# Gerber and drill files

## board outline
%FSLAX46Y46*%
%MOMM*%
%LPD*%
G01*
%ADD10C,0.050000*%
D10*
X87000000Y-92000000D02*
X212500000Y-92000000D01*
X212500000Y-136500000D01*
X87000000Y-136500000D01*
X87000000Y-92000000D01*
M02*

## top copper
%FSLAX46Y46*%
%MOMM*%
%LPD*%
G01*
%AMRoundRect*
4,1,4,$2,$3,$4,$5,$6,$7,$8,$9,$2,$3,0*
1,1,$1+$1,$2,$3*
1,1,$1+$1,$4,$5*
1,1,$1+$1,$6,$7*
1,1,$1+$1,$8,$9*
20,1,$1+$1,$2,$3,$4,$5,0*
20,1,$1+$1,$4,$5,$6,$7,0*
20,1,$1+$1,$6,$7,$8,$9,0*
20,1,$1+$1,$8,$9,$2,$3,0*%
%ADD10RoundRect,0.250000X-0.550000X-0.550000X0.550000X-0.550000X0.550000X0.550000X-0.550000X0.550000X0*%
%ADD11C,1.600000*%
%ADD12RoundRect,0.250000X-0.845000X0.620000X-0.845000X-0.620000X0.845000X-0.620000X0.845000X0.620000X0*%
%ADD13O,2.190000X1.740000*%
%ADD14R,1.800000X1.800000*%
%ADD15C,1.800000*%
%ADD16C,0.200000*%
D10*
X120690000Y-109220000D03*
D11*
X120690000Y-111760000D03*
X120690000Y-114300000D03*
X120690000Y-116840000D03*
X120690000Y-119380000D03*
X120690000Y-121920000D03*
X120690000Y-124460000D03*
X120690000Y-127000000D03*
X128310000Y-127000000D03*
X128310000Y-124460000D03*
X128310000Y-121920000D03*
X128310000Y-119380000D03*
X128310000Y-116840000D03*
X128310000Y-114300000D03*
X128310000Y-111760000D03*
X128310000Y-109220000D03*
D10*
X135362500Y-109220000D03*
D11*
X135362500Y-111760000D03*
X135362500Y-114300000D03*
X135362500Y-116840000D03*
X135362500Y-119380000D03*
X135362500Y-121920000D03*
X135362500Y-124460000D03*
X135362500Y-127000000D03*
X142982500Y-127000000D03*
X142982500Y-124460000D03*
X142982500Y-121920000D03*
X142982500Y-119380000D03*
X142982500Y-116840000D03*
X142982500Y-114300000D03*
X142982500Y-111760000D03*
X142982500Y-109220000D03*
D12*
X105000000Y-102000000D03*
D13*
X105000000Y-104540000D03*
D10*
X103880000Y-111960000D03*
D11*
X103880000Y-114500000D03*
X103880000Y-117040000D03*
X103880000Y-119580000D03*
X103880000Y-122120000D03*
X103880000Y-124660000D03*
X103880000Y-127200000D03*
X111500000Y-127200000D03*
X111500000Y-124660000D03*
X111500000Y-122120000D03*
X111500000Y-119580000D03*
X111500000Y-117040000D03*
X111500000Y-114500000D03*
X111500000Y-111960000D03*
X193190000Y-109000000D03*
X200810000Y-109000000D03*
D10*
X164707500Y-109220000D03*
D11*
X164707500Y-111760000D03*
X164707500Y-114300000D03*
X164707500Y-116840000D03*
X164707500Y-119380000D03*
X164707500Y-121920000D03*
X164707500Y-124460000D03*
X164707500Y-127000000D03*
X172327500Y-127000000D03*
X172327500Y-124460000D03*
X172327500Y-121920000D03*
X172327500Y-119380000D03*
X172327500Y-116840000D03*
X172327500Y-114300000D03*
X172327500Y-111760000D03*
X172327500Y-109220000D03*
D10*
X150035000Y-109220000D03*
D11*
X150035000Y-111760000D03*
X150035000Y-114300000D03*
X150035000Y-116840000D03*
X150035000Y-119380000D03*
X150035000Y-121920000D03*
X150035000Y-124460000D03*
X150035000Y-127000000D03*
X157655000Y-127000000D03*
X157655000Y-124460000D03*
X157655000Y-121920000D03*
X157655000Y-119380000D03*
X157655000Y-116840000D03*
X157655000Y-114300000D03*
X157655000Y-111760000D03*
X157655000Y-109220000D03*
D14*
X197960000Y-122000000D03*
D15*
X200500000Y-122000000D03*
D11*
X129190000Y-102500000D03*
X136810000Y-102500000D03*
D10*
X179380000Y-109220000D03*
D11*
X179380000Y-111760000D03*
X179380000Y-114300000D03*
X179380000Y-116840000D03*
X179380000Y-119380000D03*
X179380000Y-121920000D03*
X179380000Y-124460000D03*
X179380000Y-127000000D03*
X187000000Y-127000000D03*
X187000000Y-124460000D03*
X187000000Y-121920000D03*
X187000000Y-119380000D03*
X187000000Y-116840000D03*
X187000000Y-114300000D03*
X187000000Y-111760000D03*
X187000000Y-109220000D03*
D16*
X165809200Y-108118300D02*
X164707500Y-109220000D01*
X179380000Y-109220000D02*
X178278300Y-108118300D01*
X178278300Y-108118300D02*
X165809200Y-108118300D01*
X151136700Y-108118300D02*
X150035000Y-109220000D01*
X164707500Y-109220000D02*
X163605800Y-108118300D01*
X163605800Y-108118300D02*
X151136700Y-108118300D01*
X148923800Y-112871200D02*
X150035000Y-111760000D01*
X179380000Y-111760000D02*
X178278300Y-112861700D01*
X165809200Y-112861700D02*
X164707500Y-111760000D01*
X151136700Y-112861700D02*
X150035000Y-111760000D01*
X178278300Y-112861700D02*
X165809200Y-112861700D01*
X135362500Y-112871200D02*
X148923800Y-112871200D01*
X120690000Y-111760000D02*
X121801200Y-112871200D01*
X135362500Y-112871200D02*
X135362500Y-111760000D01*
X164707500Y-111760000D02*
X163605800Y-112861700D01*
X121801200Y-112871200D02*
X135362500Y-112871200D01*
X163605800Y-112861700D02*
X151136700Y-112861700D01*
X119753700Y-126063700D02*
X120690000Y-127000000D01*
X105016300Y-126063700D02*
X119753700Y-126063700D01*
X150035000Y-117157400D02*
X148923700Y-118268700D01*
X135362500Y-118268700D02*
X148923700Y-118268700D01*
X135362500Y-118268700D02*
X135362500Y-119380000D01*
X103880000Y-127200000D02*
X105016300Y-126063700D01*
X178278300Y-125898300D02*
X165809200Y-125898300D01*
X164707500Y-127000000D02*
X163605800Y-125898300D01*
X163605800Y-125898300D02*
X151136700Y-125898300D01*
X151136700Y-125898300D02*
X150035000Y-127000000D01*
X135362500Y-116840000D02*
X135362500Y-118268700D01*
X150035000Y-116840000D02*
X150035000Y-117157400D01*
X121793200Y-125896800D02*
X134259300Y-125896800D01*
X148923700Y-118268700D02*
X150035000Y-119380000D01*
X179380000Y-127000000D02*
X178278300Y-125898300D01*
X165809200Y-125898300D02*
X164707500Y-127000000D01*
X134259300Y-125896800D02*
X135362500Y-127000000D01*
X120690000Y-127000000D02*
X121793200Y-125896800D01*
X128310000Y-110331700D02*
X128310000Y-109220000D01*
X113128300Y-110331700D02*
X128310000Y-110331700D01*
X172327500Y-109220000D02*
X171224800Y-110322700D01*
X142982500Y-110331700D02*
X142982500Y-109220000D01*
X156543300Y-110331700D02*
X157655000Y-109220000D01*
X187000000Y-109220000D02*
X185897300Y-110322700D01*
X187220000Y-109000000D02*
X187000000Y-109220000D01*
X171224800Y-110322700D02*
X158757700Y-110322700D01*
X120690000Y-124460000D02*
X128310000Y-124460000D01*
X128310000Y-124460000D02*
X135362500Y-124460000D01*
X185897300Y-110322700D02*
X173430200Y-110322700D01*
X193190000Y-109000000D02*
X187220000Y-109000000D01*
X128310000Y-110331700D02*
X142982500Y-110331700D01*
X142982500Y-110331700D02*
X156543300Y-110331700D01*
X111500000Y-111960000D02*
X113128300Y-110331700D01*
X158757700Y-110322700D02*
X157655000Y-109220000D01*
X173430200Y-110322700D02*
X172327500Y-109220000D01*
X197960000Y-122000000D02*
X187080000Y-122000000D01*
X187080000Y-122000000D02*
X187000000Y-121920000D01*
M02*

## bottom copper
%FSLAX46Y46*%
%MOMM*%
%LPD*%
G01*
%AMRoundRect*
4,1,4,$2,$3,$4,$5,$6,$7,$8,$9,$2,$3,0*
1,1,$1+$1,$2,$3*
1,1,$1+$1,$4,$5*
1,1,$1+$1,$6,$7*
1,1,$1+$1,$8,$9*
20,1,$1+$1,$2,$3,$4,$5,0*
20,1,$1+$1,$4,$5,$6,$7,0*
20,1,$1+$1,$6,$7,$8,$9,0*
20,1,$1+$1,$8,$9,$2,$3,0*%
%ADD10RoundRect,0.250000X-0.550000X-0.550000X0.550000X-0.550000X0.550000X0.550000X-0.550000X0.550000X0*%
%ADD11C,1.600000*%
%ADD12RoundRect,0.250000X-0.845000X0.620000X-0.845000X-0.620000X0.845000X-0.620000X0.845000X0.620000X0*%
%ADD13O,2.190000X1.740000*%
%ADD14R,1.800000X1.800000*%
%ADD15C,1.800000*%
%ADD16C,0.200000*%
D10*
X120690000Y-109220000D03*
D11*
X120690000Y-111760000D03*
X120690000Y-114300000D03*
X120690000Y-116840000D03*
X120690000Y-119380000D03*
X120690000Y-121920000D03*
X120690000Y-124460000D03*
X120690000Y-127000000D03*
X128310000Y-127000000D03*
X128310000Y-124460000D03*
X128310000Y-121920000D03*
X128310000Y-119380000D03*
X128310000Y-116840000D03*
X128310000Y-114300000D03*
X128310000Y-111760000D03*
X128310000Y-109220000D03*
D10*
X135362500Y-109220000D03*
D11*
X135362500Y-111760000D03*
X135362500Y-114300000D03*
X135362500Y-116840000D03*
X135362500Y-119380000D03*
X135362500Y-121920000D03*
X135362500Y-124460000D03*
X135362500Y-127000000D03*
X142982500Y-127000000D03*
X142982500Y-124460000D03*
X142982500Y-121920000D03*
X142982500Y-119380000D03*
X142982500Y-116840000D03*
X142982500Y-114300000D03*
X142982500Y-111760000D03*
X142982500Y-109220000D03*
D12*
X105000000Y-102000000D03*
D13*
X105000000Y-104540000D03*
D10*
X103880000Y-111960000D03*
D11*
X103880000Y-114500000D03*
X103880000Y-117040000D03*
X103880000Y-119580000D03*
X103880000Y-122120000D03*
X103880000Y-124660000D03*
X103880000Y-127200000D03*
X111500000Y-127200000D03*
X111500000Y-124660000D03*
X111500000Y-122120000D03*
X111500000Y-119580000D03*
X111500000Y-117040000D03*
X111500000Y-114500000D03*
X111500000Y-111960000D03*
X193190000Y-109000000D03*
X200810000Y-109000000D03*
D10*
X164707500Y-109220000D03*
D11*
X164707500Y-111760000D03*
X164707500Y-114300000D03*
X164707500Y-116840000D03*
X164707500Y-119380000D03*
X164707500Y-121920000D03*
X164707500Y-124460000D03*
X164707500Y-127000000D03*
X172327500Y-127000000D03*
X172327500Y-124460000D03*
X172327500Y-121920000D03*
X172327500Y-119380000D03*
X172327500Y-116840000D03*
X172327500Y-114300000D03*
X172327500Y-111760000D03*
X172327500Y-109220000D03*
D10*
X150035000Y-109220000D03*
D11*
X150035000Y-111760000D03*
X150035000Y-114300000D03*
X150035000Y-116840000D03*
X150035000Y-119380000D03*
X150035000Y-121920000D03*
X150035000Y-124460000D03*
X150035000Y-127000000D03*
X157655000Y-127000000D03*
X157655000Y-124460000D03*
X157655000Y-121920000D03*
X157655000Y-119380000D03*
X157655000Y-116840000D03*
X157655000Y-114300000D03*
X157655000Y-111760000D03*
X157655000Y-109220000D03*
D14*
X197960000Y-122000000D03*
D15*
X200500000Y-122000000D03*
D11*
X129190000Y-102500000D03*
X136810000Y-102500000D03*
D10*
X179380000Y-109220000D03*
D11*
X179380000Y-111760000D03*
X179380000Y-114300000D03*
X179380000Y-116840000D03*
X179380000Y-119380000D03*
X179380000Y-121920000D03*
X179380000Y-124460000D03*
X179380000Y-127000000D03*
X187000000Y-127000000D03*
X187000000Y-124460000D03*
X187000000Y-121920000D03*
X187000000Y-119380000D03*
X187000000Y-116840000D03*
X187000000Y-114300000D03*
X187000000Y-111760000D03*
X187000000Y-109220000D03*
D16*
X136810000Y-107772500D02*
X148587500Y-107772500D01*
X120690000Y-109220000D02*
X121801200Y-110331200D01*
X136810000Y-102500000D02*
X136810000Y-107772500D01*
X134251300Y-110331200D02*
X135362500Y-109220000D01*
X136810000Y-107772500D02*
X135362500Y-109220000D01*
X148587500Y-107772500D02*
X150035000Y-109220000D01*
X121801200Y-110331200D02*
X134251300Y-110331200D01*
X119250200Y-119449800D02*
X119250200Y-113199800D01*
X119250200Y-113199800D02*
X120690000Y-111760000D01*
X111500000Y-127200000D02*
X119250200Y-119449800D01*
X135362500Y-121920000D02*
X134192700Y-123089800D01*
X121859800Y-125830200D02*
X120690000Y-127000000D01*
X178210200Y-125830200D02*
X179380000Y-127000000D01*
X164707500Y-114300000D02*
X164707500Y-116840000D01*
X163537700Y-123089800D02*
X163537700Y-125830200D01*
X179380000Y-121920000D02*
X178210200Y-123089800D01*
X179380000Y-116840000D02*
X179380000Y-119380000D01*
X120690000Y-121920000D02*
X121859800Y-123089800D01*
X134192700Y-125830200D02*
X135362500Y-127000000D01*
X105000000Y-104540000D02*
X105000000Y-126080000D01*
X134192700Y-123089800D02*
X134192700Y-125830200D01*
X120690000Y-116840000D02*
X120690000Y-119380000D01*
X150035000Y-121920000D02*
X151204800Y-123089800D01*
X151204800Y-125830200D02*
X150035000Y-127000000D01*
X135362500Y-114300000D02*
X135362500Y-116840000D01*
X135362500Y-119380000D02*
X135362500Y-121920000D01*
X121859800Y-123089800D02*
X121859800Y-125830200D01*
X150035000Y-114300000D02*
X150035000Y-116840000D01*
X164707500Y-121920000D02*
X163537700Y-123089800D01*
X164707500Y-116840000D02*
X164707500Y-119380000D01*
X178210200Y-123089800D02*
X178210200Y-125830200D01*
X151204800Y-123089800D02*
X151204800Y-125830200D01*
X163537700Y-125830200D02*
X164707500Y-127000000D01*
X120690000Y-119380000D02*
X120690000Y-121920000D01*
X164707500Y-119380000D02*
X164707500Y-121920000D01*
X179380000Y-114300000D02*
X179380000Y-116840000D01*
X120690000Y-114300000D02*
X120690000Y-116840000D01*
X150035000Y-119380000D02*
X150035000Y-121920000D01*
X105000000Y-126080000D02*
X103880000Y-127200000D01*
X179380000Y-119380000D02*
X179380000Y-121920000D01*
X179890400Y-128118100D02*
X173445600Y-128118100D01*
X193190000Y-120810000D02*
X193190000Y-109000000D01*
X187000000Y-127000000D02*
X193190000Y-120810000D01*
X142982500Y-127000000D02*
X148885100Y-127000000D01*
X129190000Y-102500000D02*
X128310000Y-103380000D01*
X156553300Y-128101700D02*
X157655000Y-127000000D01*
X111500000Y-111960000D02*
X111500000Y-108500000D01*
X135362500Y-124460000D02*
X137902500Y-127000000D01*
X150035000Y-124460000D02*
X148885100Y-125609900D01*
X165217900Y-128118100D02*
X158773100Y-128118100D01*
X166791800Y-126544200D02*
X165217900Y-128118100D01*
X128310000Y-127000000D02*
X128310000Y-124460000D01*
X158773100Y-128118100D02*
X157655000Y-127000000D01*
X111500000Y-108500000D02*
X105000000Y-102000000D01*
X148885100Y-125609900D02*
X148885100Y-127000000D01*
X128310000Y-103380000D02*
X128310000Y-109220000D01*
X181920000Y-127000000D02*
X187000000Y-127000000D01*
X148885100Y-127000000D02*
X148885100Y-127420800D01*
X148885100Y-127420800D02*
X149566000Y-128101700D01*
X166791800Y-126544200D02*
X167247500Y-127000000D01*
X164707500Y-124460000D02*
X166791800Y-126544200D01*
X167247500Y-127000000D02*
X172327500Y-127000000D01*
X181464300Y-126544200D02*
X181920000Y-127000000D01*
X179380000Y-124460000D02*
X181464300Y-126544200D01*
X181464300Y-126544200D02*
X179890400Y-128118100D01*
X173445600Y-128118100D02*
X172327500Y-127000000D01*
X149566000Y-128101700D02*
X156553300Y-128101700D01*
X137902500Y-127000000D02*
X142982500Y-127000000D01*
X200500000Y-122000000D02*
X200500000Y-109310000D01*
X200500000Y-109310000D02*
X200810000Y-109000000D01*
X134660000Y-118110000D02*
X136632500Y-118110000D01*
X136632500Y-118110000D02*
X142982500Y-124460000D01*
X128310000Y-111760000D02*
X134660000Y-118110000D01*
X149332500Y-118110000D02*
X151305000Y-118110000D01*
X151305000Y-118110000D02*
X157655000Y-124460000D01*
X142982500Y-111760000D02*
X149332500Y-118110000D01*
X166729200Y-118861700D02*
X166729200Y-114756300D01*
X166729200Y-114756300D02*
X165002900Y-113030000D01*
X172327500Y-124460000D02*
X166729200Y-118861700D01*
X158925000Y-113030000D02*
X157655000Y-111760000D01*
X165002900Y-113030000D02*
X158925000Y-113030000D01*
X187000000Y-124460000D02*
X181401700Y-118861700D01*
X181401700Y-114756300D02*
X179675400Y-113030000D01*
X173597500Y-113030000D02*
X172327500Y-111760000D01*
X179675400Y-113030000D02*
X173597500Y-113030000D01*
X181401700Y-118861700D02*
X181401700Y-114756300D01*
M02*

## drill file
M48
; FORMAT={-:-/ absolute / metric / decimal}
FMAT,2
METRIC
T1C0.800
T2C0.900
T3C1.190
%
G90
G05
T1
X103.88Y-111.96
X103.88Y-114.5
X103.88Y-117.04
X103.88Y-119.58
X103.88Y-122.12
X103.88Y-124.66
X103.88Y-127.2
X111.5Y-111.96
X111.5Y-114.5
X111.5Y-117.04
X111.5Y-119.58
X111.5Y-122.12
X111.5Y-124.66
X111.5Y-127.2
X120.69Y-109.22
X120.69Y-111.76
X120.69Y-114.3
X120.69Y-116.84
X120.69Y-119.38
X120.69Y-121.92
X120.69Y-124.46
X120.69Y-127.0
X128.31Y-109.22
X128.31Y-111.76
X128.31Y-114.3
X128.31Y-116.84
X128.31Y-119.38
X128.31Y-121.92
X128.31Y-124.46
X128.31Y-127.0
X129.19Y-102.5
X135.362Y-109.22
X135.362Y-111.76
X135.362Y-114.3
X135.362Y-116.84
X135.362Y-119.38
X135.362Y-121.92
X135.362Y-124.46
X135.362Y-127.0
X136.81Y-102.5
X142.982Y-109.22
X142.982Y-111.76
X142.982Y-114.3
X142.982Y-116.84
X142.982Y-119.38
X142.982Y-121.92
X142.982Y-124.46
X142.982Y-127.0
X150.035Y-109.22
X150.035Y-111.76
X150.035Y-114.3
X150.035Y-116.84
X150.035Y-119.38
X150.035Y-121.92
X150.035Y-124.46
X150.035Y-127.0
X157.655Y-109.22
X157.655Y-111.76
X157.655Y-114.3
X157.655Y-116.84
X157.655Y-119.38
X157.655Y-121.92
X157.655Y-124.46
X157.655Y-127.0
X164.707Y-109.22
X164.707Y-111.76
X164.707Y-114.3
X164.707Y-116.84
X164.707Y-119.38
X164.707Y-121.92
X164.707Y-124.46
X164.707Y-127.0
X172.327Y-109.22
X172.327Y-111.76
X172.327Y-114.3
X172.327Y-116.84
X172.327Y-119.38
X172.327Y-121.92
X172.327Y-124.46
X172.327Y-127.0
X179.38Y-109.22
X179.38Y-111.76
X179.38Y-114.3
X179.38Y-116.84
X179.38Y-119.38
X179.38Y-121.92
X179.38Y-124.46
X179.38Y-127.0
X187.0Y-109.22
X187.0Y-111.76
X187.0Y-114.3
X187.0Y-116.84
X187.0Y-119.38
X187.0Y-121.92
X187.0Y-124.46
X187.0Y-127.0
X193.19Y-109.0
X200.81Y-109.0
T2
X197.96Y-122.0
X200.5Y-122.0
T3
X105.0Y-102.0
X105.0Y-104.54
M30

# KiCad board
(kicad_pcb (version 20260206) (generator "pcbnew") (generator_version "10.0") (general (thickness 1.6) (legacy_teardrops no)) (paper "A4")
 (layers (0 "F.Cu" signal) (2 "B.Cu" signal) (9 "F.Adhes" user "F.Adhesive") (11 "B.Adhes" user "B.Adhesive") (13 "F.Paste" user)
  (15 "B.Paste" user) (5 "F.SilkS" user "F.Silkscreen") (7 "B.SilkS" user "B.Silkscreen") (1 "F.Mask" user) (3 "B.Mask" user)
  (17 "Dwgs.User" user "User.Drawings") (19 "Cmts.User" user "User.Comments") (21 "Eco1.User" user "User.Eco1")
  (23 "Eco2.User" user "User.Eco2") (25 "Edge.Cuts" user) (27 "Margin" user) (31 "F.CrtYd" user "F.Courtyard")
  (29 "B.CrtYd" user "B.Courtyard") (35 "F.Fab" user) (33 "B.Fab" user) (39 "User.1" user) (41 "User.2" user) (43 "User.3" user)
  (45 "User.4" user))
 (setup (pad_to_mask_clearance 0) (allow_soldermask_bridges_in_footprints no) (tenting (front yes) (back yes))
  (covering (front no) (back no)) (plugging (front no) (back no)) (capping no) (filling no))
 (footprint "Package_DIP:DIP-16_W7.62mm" (layer "F.Cu") (at 120.69 109.22)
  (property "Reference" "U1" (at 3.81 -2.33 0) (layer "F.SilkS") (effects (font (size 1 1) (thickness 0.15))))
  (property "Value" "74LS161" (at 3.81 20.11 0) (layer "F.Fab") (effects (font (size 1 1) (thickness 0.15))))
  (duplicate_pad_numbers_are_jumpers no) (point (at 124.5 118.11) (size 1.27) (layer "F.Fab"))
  (pad "1" thru_hole roundrect (at 0 0) (size 1.6 1.6) (drill 0.8) (layers "*.Cu" "*.Mask") (remove_unused_layers no)
   (roundrect_rratio 0.15625) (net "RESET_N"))
  (pad "2" thru_hole circle (at 0 2.54) (size 1.6 1.6) (drill 0.8) (layers "*.Cu" "*.Mask") (remove_unused_layers no) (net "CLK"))
  (pad "3" thru_hole circle (at 0 5.08) (size 1.6 1.6) (drill 0.8) (layers "*.Cu" "*.Mask") (remove_unused_layers no) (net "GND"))
  (pad "4" thru_hole circle (at 0 7.62) (size 1.6 1.6) (drill 0.8) (layers "*.Cu" "*.Mask") (remove_unused_layers no) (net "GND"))
  (pad "5" thru_hole circle (at 0 10.16) (size 1.6 1.6) (drill 0.8) (layers "*.Cu" "*.Mask") (remove_unused_layers no) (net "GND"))
  (pad "6" thru_hole circle (at 0 12.7) (size 1.6 1.6) (drill 0.8) (layers "*.Cu" "*.Mask") (remove_unused_layers no) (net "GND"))
  (pad "7" thru_hole circle (at 0 15.24) (size 1.6 1.6) (drill 0.8) (layers "*.Cu" "*.Mask") (remove_unused_layers no) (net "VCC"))
  (pad "8" thru_hole circle (at 0 17.78) (size 1.6 1.6) (drill 0.8) (layers "*.Cu" "*.Mask") (remove_unused_layers no) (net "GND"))
  (pad "9" thru_hole circle (at 7.62 17.78) (size 1.6 1.6) (drill 0.8) (layers "*.Cu" "*.Mask") (remove_unused_layers no) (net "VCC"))
  (pad "10" thru_hole circle (at 7.62 15.24) (size 1.6 1.6) (drill 0.8) (layers "*.Cu" "*.Mask") (remove_unused_layers no) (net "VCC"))
  (pad "11" thru_hole circle (at 7.62 12.7) (size 1.6 1.6) (drill 0.8) (layers "*.Cu" "*.Mask") (remove_unused_layers no) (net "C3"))
  (pad "12" thru_hole circle (at 7.62 10.16) (size 1.6 1.6) (drill 0.8) (layers "*.Cu" "*.Mask") (remove_unused_layers no) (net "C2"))
  (pad "13" thru_hole circle (at 7.62 7.62) (size 1.6 1.6) (drill 0.8) (layers "*.Cu" "*.Mask") (remove_unused_layers no) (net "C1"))
  (pad "14" thru_hole circle (at 7.62 5.08) (size 1.6 1.6) (drill 0.8) (layers "*.Cu" "*.Mask") (remove_unused_layers no) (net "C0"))
  (pad "15" thru_hole circle (at 7.62 2.54) (size 1.6 1.6) (drill 0.8) (layers "*.Cu" "*.Mask") (remove_unused_layers no) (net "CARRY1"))
  (pad "16" thru_hole circle (at 7.62 0) (size 1.6 1.6) (drill 0.8) (layers "*.Cu" "*.Mask") (remove_unused_layers no) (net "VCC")))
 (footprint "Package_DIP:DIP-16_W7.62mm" (layer "F.Cu") (at 135.3625 109.22)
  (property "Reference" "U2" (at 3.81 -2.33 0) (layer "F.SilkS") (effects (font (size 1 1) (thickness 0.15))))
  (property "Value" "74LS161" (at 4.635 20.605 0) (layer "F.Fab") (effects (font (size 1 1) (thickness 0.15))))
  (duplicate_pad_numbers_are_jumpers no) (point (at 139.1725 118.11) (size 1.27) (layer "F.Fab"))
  (pad "1" thru_hole roundrect (at 0 0) (size 1.6 1.6) (drill 0.8) (layers "*.Cu" "*.Mask") (remove_unused_layers no)
   (roundrect_rratio 0.15625) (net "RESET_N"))
  (pad "2" thru_hole circle (at 0 2.54) (size 1.6 1.6) (drill 0.8) (layers "*.Cu" "*.Mask") (remove_unused_layers no) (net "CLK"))
  (pad "3" thru_hole circle (at 0 5.08) (size 1.6 1.6) (drill 0.8) (layers "*.Cu" "*.Mask") (remove_unused_layers no) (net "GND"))
  (pad "4" thru_hole circle (at 0 7.62) (size 1.6 1.6) (drill 0.8) (layers "*.Cu" "*.Mask") (remove_unused_layers no) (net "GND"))
  (pad "5" thru_hole circle (at 0 10.16) (size 1.6 1.6) (drill 0.8) (layers "*.Cu" "*.Mask") (remove_unused_layers no) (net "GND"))
  (pad "6" thru_hole circle (at 0 12.7) (size 1.6 1.6) (drill 0.8) (layers "*.Cu" "*.Mask") (remove_unused_layers no) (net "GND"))
  (pad "7" thru_hole circle (at 0 15.24) (size 1.6 1.6) (drill 0.8) (layers "*.Cu" "*.Mask") (remove_unused_layers no) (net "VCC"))
  (pad "8" thru_hole circle (at 0 17.78) (size 1.6 1.6) (drill 0.8) (layers "*.Cu" "*.Mask") (remove_unused_layers no) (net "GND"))
  (pad "9" thru_hole circle (at 7.62 17.78) (size 1.6 1.6) (drill 0.8) (layers "*.Cu" "*.Mask") (remove_unused_layers no) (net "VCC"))
  (pad "10" thru_hole circle (at 7.62 15.24) (size 1.6 1.6) (drill 0.8) (layers "*.Cu" "*.Mask") (remove_unused_layers no) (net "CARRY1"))
  (pad "11" thru_hole circle (at 7.62 12.7) (size 1.6 1.6) (drill 0.8) (layers "*.Cu" "*.Mask") (remove_unused_layers no) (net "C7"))
  (pad "12" thru_hole circle (at 7.62 10.16) (size 1.6 1.6) (drill 0.8) (layers "*.Cu" "*.Mask") (remove_unused_layers no) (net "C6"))
  (pad "13" thru_hole circle (at 7.62 7.62) (size 1.6 1.6) (drill 0.8) (layers "*.Cu" "*.Mask") (remove_unused_layers no) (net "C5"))
  (pad "14" thru_hole circle (at 7.62 5.08) (size 1.6 1.6) (drill 0.8) (layers "*.Cu" "*.Mask") (remove_unused_layers no) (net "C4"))
  (pad "15" thru_hole circle (at 7.62 2.54) (size 1.6 1.6) (drill 0.8) (layers "*.Cu" "*.Mask") (remove_unused_layers no) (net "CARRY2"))
  (pad "16" thru_hole circle (at 7.62 0) (size 1.6 1.6) (drill 0.8) (layers "*.Cu" "*.Mask") (remove_unused_layers no) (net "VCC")))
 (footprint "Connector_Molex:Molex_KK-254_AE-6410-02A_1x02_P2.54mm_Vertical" (layer "F.Cu") (at 105 102 -90)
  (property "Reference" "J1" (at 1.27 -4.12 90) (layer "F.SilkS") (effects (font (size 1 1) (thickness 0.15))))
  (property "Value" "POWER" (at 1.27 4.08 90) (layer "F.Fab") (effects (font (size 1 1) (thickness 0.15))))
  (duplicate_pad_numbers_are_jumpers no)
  (pad "1" thru_hole roundrect (at 0 0 270) (size 1.74 2.19) (drill 1.19) (layers "*.Cu" "*.Mask") (remove_unused_layers no)
   (roundrect_rratio 0.143678) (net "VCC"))
  (pad "2" thru_hole oval (at 2.54 0 270) (size 1.74 2.19) (drill 1.19) (layers "*.Cu" "*.Mask") (remove_unused_layers no) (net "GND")))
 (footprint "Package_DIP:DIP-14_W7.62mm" (layer "F.Cu") (at 103.88 111.96)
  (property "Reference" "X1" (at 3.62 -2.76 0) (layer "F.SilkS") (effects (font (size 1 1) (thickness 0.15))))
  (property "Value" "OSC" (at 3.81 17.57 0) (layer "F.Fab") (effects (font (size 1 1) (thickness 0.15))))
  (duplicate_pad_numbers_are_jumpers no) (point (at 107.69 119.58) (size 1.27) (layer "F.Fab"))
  (pad "1" thru_hole roundrect (at 0 0) (size 1.6 1.6) (drill 0.8) (layers "*.Cu" "*.Mask") (remove_unused_layers no)
   (roundrect_rratio 0.15625))
  (pad "2" thru_hole circle (at 0 2.54) (size 1.6 1.6) (drill 0.8) (layers "*.Cu" "*.Mask") (remove_unused_layers no))
  (pad "3" thru_hole circle (at 0 5.08) (size 1.6 1.6) (drill 0.8) (layers "*.Cu" "*.Mask") (remove_unused_layers no))
  (pad "4" thru_hole circle (at 0 7.62) (size 1.6 1.6) (drill 0.8) (layers "*.Cu" "*.Mask") (remove_unused_layers no))
  (pad "5" thru_hole circle (at 0 10.16) (size 1.6 1.6) (drill 0.8) (layers "*.Cu" "*.Mask") (remove_unused_layers no))
  (pad "6" thru_hole circle (at 0 12.7) (size 1.6 1.6) (drill 0.8) (layers "*.Cu" "*.Mask") (remove_unused_layers no))
  (pad "7" thru_hole circle (at 0 15.24) (size 1.6 1.6) (drill 0.8) (layers "*.Cu" "*.Mask") (remove_unused_layers no) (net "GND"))
  (pad "8" thru_hole circle (at 7.62 15.24) (size 1.6 1.6) (drill 0.8) (layers "*.Cu" "*.Mask") (remove_unused_layers no) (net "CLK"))
  (pad "9" thru_hole circle (at 7.62 12.7) (size 1.6 1.6) (drill 0.8) (layers "*.Cu" "*.Mask") (remove_unused_layers no))
  (pad "10" thru_hole circle (at 7.62 10.16) (size 1.6 1.6) (drill 0.8) (layers "*.Cu" "*.Mask") (remove_unused_layers no))
  (pad "11" thru_hole circle (at 7.62 7.62) (size 1.6 1.6) (drill 0.8) (layers "*.Cu" "*.Mask") (remove_unused_layers no))
  (pad "12" thru_hole circle (at 7.62 5.08) (size 1.6 1.6) (drill 0.8) (layers "*.Cu" "*.Mask") (remove_unused_layers no))
  (pad "13" thru_hole circle (at 7.62 2.54) (size 1.6 1.6) (drill 0.8) (layers "*.Cu" "*.Mask") (remove_unused_layers no))
  (pad "14" thru_hole circle (at 7.62 0) (size 1.6 1.6) (drill 0.8) (layers "*.Cu" "*.Mask") (remove_unused_layers no) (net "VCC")))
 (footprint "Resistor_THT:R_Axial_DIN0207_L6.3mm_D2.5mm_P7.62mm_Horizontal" (layer "F.Cu") (at 193.19 109)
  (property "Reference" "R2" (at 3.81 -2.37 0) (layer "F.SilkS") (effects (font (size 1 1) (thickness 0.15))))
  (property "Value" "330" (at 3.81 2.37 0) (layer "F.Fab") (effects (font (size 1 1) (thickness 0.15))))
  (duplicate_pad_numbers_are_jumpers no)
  (pad "1" thru_hole circle (at 0 0) (size 1.6 1.6) (drill 0.8) (layers "*.Cu" "*.Mask") (remove_unused_layers no) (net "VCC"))
  (pad "2" thru_hole circle (at 7.62 0) (size 1.6 1.6) (drill 0.8) (layers "*.Cu" "*.Mask") (remove_unused_layers no) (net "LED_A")))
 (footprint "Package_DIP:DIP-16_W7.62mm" (layer "F.Cu") (at 164.7075 109.22)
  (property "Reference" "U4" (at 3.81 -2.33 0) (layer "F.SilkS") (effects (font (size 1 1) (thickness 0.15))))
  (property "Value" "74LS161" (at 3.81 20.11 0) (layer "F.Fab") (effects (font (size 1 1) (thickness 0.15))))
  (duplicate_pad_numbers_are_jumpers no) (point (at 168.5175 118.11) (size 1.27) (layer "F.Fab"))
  (pad "1" thru_hole roundrect (at 0 0) (size 1.6 1.6) (drill 0.8) (layers "*.Cu" "*.Mask") (remove_unused_layers no)
   (roundrect_rratio 0.15625) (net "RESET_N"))
  (pad "2" thru_hole circle (at 0 2.54) (size 1.6 1.6) (drill 0.8) (layers "*.Cu" "*.Mask") (remove_unused_layers no) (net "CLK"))
  (pad "3" thru_hole circle (at 0 5.08) (size 1.6 1.6) (drill 0.8) (layers "*.Cu" "*.Mask") (remove_unused_layers no) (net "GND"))
  (pad "4" thru_hole circle (at 0 7.62) (size 1.6 1.6) (drill 0.8) (layers "*.Cu" "*.Mask") (remove_unused_layers no) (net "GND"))
  (pad "5" thru_hole circle (at 0 10.16) (size 1.6 1.6) (drill 0.8) (layers "*.Cu" "*.Mask") (remove_unused_layers no) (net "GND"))
  (pad "6" thru_hole circle (at 0 12.7) (size 1.6 1.6) (drill 0.8) (layers "*.Cu" "*.Mask") (remove_unused_layers no) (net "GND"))
  (pad "7" thru_hole circle (at 0 15.24) (size 1.6 1.6) (drill 0.8) (layers "*.Cu" "*.Mask") (remove_unused_layers no) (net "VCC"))
  (pad "8" thru_hole circle (at 0 17.78) (size 1.6 1.6) (drill 0.8) (layers "*.Cu" "*.Mask") (remove_unused_layers no) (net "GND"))
  (pad "9" thru_hole circle (at 7.62 17.78) (size 1.6 1.6) (drill 0.8) (layers "*.Cu" "*.Mask") (remove_unused_layers no) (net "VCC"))
  (pad "10" thru_hole circle (at 7.62 15.24) (size 1.6 1.6) (drill 0.8) (layers "*.Cu" "*.Mask") (remove_unused_layers no) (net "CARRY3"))
  (pad "11" thru_hole circle (at 7.62 12.7) (size 1.6 1.6) (drill 0.8) (layers "*.Cu" "*.Mask") (remove_unused_layers no) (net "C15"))
  (pad "12" thru_hole circle (at 7.62 10.16) (size 1.6 1.6) (drill 0.8) (layers "*.Cu" "*.Mask") (remove_unused_layers no) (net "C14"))
  (pad "13" thru_hole circle (at 7.62 7.62) (size 1.6 1.6) (drill 0.8) (layers "*.Cu" "*.Mask") (remove_unused_layers no) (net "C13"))
  (pad "14" thru_hole circle (at 7.62 5.08) (size 1.6 1.6) (drill 0.8) (layers "*.Cu" "*.Mask") (remove_unused_layers no) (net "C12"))
  (pad "15" thru_hole circle (at 7.62 2.54) (size 1.6 1.6) (drill 0.8) (layers "*.Cu" "*.Mask") (remove_unused_layers no) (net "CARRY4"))
  (pad "16" thru_hole circle (at 7.62 0) (size 1.6 1.6) (drill 0.8) (layers "*.Cu" "*.Mask") (remove_unused_layers no) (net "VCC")))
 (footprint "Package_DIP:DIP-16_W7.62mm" (layer "F.Cu") (at 150.035 109.22)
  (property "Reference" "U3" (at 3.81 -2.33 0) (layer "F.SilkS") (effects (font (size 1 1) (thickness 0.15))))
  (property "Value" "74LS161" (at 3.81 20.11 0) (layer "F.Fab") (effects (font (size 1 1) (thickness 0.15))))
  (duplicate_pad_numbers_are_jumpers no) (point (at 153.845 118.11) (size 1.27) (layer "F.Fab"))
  (pad "1" thru_hole roundrect (at 0 0) (size 1.6 1.6) (drill 0.8) (layers "*.Cu" "*.Mask") (remove_unused_layers no)
   (roundrect_rratio 0.15625) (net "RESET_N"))
  (pad "2" thru_hole circle (at 0 2.54) (size 1.6 1.6) (drill 0.8) (layers "*.Cu" "*.Mask") (remove_unused_layers no) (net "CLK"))
  (pad "3" thru_hole circle (at 0 5.08) (size 1.6 1.6) (drill 0.8) (layers "*.Cu" "*.Mask") (remove_unused_layers no) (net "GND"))
  (pad "4" thru_hole circle (at 0 7.62) (size 1.6 1.6) (drill 0.8) (layers "*.Cu" "*.Mask") (remove_unused_layers no) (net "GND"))
  (pad "5" thru_hole circle (at 0 10.16) (size 1.6 1.6) (drill 0.8) (layers "*.Cu" "*.Mask") (remove_unused_layers no) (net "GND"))
  (pad "6" thru_hole circle (at 0 12.7) (size 1.6 1.6) (drill 0.8) (layers "*.Cu" "*.Mask") (remove_unused_layers no) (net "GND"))
  (pad "7" thru_hole circle (at 0 15.24) (size 1.6 1.6) (drill 0.8) (layers "*.Cu" "*.Mask") (remove_unused_layers no) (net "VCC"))
  (pad "8" thru_hole circle (at 0 17.78) (size 1.6 1.6) (drill 0.8) (layers "*.Cu" "*.Mask") (remove_unused_layers no) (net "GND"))
  (pad "9" thru_hole circle (at 7.62 17.78) (size 1.6 1.6) (drill 0.8) (layers "*.Cu" "*.Mask") (remove_unused_layers no) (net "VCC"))
  (pad "10" thru_hole circle (at 7.62 15.24) (size 1.6 1.6) (drill 0.8) (layers "*.Cu" "*.Mask") (remove_unused_layers no) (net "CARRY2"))
  (pad "11" thru_hole circle (at 7.62 12.7) (size 1.6 1.6) (drill 0.8) (layers "*.Cu" "*.Mask") (remove_unused_layers no) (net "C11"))
  (pad "12" thru_hole circle (at 7.62 10.16) (size 1.6 1.6) (drill 0.8) (layers "*.Cu" "*.Mask") (remove_unused_layers no) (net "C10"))
  (pad "13" thru_hole circle (at 7.62 7.62) (size 1.6 1.6) (drill 0.8) (layers "*.Cu" "*.Mask") (remove_unused_layers no) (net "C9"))
  (pad "14" thru_hole circle (at 7.62 5.08) (size 1.6 1.6) (drill 0.8) (layers "*.Cu" "*.Mask") (remove_unused_layers no) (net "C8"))
  (pad "15" thru_hole circle (at 7.62 2.54) (size 1.6 1.6) (drill 0.8) (layers "*.Cu" "*.Mask") (remove_unused_layers no) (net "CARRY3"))
  (pad "16" thru_hole circle (at 7.62 0) (size 1.6 1.6) (drill 0.8) (layers "*.Cu" "*.Mask") (remove_unused_layers no) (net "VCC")))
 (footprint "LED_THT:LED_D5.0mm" (layer "F.Cu") (at 197.96 122)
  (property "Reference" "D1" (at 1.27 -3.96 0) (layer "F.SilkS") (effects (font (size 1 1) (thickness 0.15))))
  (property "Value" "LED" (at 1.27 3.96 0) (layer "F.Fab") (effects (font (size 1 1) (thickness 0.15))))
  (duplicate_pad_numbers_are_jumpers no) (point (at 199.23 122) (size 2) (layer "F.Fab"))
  (pad "1" thru_hole rect (at 0 0) (size 1.8 1.8) (drill 0.9) (layers "*.Cu" "*.Mask") (remove_unused_layers no) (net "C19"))
  (pad "2" thru_hole circle (at 2.54 0) (size 1.8 1.8) (drill 0.9) (layers "*.Cu" "*.Mask") (remove_unused_layers no) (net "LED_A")))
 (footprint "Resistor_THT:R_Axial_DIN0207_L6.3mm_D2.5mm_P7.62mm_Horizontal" (layer "F.Cu") (at 129.19 102.5)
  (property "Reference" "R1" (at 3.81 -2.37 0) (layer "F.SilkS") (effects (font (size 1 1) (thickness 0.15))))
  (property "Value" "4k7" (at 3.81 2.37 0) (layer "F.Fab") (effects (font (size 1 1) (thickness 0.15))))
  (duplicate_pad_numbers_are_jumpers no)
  (pad "1" thru_hole circle (at 0 0) (size 1.6 1.6) (drill 0.8) (layers "*.Cu" "*.Mask") (remove_unused_layers no) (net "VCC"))
  (pad "2" thru_hole circle (at 7.62 0) (size 1.6 1.6) (drill 0.8) (layers "*.Cu" "*.Mask") (remove_unused_layers no) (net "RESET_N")))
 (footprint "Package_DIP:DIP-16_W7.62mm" (layer "F.Cu") (at 179.38 109.22)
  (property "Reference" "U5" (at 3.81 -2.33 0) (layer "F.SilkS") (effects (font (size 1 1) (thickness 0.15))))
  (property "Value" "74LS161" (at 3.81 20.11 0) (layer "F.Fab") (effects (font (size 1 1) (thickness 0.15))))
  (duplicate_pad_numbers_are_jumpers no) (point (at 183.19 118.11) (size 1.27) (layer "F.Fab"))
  (pad "1" thru_hole roundrect (at 0 0) (size 1.6 1.6) (drill 0.8) (layers "*.Cu" "*.Mask") (remove_unused_layers no)
   (roundrect_rratio 0.15625) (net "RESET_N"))
  (pad "2" thru_hole circle (at 0 2.54) (size 1.6 1.6) (drill 0.8) (layers "*.Cu" "*.Mask") (remove_unused_layers no) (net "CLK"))
  (pad "3" thru_hole circle (at 0 5.08) (size 1.6 1.6) (drill 0.8) (layers "*.Cu" "*.Mask") (remove_unused_layers no) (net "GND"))
  (pad "4" thru_hole circle (at 0 7.62) (size 1.6 1.6) (drill 0.8) (layers "*.Cu" "*.Mask") (remove_unused_layers no) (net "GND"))
  (pad "5" thru_hole circle (at 0 10.16) (size 1.6 1.6) (drill 0.8) (layers "*.Cu" "*.Mask") (remove_unused_layers no) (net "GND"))
  (pad "6" thru_hole circle (at 0 12.7) (size 1.6 1.6) (drill 0.8) (layers "*.Cu" "*.Mask") (remove_unused_layers no) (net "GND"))
  (pad "7" thru_hole circle (at 0 15.24) (size 1.6 1.6) (drill 0.8) (layers "*.Cu" "*.Mask") (remove_unused_layers no) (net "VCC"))
  (pad "8" thru_hole circle (at 0 17.78) (size 1.6 1.6) (drill 0.8) (layers "*.Cu" "*.Mask") (remove_unused_layers no) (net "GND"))
  (pad "9" thru_hole circle (at 7.62 17.78) (size 1.6 1.6) (drill 0.8) (layers "*.Cu" "*.Mask") (remove_unused_layers no) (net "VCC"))
  (pad "10" thru_hole circle (at 7.62 15.24) (size 1.6 1.6) (drill 0.8) (layers "*.Cu" "*.Mask") (remove_unused_layers no) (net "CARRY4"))
  (pad "11" thru_hole circle (at 7.62 12.7) (size 1.6 1.6) (drill 0.8) (layers "*.Cu" "*.Mask") (remove_unused_layers no) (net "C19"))
  (pad "12" thru_hole circle (at 7.62 10.16) (size 1.6 1.6) (drill 0.8) (layers "*.Cu" "*.Mask") (remove_unused_layers no) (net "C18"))
  (pad "13" thru_hole circle (at 7.62 7.62) (size 1.6 1.6) (drill 0.8) (layers "*.Cu" "*.Mask") (remove_unused_layers no) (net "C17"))
  (pad "14" thru_hole circle (at 7.62 5.08) (size 1.6 1.6) (drill 0.8) (layers "*.Cu" "*.Mask") (remove_unused_layers no) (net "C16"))
  (pad "15" thru_hole circle (at 7.62 2.54) (size 1.6 1.6) (drill 0.8) (layers "*.Cu" "*.Mask") (remove_unused_layers no))
  (pad "16" thru_hole circle (at 7.62 0) (size 1.6 1.6) (drill 0.8) (layers "*.Cu" "*.Mask") (remove_unused_layers no) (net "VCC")))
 (gr_rect (start 87 92) (end 212.5 136.5) (stroke (width 0.05) (type default)) (fill no) (layer "Edge.Cuts"))
 (segment (start 165.8092 108.1183) (end 164.7075 109.22) (width 0.2) (layer "F.Cu") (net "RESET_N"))
 (segment (start 179.38 109.22) (end 178.2783 108.1183) (width 0.2) (layer "F.Cu") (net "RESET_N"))
 (segment (start 178.2783 108.1183) (end 165.8092 108.1183) (width 0.2) (layer "F.Cu") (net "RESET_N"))
 (segment (start 151.1367 108.1183) (end 150.035 109.22) (width 0.2) (layer "F.Cu") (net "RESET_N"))
 (segment (start 164.7075 109.22) (end 163.6058 108.1183) (width 0.2) (layer "F.Cu") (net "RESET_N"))
 (segment (start 163.6058 108.1183) (end 151.1367 108.1183) (width 0.2) (layer "F.Cu") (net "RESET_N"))
 (segment (start 136.81 107.7725) (end 148.5875 107.7725) (width 0.2) (layer "B.Cu") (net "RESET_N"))
 (segment (start 120.69 109.22) (end 121.8012 110.3312) (width 0.2) (layer "B.Cu") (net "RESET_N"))
 (segment (start 136.81 102.5) (end 136.81 107.7725) (width 0.2) (layer "B.Cu") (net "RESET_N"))
 (segment (start 134.2513 110.3312) (end 135.3625 109.22) (width 0.2) (layer "B.Cu") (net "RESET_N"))
 (segment (start 136.81 107.7725) (end 135.3625 109.22) (width 0.2) (layer "B.Cu") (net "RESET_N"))
 (segment (start 148.5875 107.7725) (end 150.035 109.22) (width 0.2) (layer "B.Cu") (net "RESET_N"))
 (segment (start 121.8012 110.3312) (end 134.2513 110.3312) (width 0.2) (layer "B.Cu") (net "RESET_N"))
 (segment (start 148.9238 112.8712) (end 150.035 111.76) (width 0.2) (layer "F.Cu") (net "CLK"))
 (segment (start 179.38 111.76) (end 178.2783 112.8617) (width 0.2) (layer "F.Cu") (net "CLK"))
 (segment (start 165.8092 112.8617) (end 164.7075 111.76) (width 0.2) (layer "F.Cu") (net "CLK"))
 (segment (start 151.1367 112.8617) (end 150.035 111.76) (width 0.2) (layer "F.Cu") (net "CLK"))
 (segment (start 178.2783 112.8617) (end 165.8092 112.8617) (width 0.2) (layer "F.Cu") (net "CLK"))
 (segment (start 135.3625 112.8712) (end 148.9238 112.8712) (width 0.2) (layer "F.Cu") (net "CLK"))
 (segment (start 120.69 111.76) (end 121.8012 112.8712) (width 0.2) (layer "F.Cu") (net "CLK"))
 (segment (start 135.3625 112.8712) (end 135.3625 111.76) (width 0.2) (layer "F.Cu") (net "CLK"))
 (segment (start 164.7075 111.76) (end 163.6058 112.8617) (width 0.2) (layer "F.Cu") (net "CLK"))
 (segment (start 121.8012 112.8712) (end 135.3625 112.8712) (width 0.2) (layer "F.Cu") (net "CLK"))
 (segment (start 163.6058 112.8617) (end 151.1367 112.8617) (width 0.2) (layer "F.Cu") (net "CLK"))
 (segment (start 119.2502 119.4498) (end 119.2502 113.1998) (width 0.2) (layer "B.Cu") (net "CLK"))
 (segment (start 119.2502 113.1998) (end 120.69 111.76) (width 0.2) (layer "B.Cu") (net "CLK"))
 (segment (start 111.5 127.2) (end 119.2502 119.4498) (width 0.2) (layer "B.Cu") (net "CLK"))
 (segment (start 119.7537 126.0637) (end 120.69 127) (width 0.2) (layer "F.Cu") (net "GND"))
 (segment (start 105.0163 126.0637) (end 119.7537 126.0637) (width 0.2) (layer "F.Cu") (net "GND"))
 (segment (start 150.035 117.1574) (end 148.9237 118.2687) (width 0.2) (layer "F.Cu") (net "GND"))
 (segment (start 135.3625 118.2687) (end 148.9237 118.2687) (width 0.2) (layer "F.Cu") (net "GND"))
 (segment (start 135.3625 118.2687) (end 135.3625 119.38) (width 0.2) (layer "F.Cu") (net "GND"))
 (segment (start 103.88 127.2) (end 105.0163 126.0637) (width 0.2) (layer "F.Cu") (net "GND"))
 (segment (start 178.2783 125.8983) (end 165.8092 125.8983) (width 0.2) (layer "F.Cu") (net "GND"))
 (segment (start 164.7075 127) (end 163.6058 125.8983) (width 0.2) (layer "F.Cu") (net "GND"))
 (segment (start 163.6058 125.8983) (end 151.1367 125.8983) (width 0.2) (layer "F.Cu") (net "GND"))
 (segment (start 151.1367 125.8983) (end 150.035 127) (width 0.2) (layer "F.Cu") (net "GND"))
 (segment (start 135.3625 116.84) (end 135.3625 118.2687) (width 0.2) (layer "F.Cu") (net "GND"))
 (segment (start 150.035 116.84) (end 150.035 117.1574) (width 0.2) (layer "F.Cu") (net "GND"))
 (segment (start 121.7932 125.8968) (end 134.2593 125.8968) (width 0.2) (layer "F.Cu") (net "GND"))
 (segment (start 148.9237 118.2687) (end 150.035 119.38) (width 0.2) (layer "F.Cu") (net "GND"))
 (segment (start 179.38 127) (end 178.2783 125.8983) (width 0.2) (layer "F.Cu") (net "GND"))
 (segment (start 165.8092 125.8983) (end 164.7075 127) (width 0.2) (layer "F.Cu") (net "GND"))
 (segment (start 134.2593 125.8968) (end 135.3625 127) (width 0.2) (layer "F.Cu") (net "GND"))
 (segment (start 120.69 127) (end 121.7932 125.8968) (width 0.2) (layer "F.Cu") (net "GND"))
 (segment (start 135.3625 121.92) (end 134.1927 123.0898) (width 0.2) (layer "B.Cu") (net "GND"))
 (segment (start 121.8598 125.8302) (end 120.69 127) (width 0.2) (layer "B.Cu") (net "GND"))
 (segment (start 178.2102 125.8302) (end 179.38 127) (width 0.2) (layer "B.Cu") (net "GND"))
 (segment (start 164.7075 114.3) (end 164.7075 116.84) (width 0.2) (layer "B.Cu") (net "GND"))
 (segment (start 163.5377 123.0898) (end 163.5377 125.8302) (width 0.2) (layer "B.Cu") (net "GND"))
 (segment (start 179.38 121.92) (end 178.2102 123.0898) (width 0.2) (layer "B.Cu") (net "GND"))
 (segment (start 179.38 116.84) (end 179.38 119.38) (width 0.2) (layer "B.Cu") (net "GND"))
 (segment (start 120.69 121.92) (end 121.8598 123.0898) (width 0.2) (layer "B.Cu") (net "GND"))
 (segment (start 134.1927 125.8302) (end 135.3625 127) (width 0.2) (layer "B.Cu") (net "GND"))
 (segment (start 105 104.54) (end 105 126.08) (width 0.2) (layer "B.Cu") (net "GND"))
 (segment (start 134.1927 123.0898) (end 134.1927 125.8302) (width 0.2) (layer "B.Cu") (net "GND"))
 (segment (start 120.69 116.84) (end 120.69 119.38) (width 0.2) (layer "B.Cu") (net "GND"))
 (segment (start 150.035 121.92) (end 151.2048 123.0898) (width 0.2) (layer "B.Cu") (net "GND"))
 (segment (start 151.2048 125.8302) (end 150.035 127) (width 0.2) (layer "B.Cu") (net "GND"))
 (segment (start 135.3625 114.3) (end 135.3625 116.84) (width 0.2) (layer "B.Cu") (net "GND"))
 (segment (start 135.3625 119.38) (end 135.3625 121.92) (width 0.2) (layer "B.Cu") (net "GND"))
 (segment (start 121.8598 123.0898) (end 121.8598 125.8302) (width 0.2) (layer "B.Cu") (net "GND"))
 (segment (start 150.035 114.3) (end 150.035 116.84) (width 0.2) (layer "B.Cu") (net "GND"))
 (segment (start 164.7075 121.92) (end 163.5377 123.0898) (width 0.2) (layer "B.Cu") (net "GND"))
 (segment (start 164.7075 116.84) (end 164.7075 119.38) (width 0.2) (layer "B.Cu") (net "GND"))
 (segment (start 178.2102 123.0898) (end 178.2102 125.8302) (width 0.2) (layer "B.Cu") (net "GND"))
 (segment (start 151.2048 123.0898) (end 151.2048 125.8302) (width 0.2) (layer "B.Cu") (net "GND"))
 (segment (start 163.5377 125.8302) (end 164.7075 127) (width 0.2) (layer "B.Cu") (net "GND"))
 (segment (start 120.69 119.38) (end 120.69 121.92) (width 0.2) (layer "B.Cu") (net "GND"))
 (segment (start 164.7075 119.38) (end 164.7075 121.92) (width 0.2) (layer "B.Cu") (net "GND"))
 (segment (start 179.38 114.3) (end 179.38 116.84) (width 0.2) (layer "B.Cu") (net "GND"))
 (segment (start 120.69 114.3) (end 120.69 116.84) (width 0.2) (layer "B.Cu") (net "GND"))
 (segment (start 150.035 119.38) (end 150.035 121.92) (width 0.2) (layer "B.Cu") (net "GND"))
 (segment (start 105 126.08) (end 103.88 127.2) (width 0.2) (layer "B.Cu") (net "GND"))
 (segment (start 179.38 119.38) (end 179.38 121.92) (width 0.2) (layer "B.Cu") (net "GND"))
 (segment (start 128.31 110.3317) (end 128.31 109.22) (width 0.2) (layer "F.Cu") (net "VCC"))
 (segment (start 113.1283 110.3317) (end 128.31 110.3317) (width 0.2) (layer "F.Cu") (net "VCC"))
 (segment (start 172.3275 109.22) (end 171.2248 110.3227) (width 0.2) (layer "F.Cu") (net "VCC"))
 (segment (start 142.9825 110.3317) (end 142.9825 109.22) (width 0.2) (layer "F.Cu") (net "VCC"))
 (segment (start 156.5433 110.3317) (end 157.655 109.22) (width 0.2) (layer "F.Cu") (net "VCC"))
 (segment (start 187 109.22) (end 185.8973 110.3227) (width 0.2) (layer "F.Cu") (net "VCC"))
 (segment (start 187.22 109) (end 187 109.22) (width 0.2) (layer "F.Cu") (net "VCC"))
 (segment (start 171.2248 110.3227) (end 158.7577 110.3227) (width 0.2) (layer "F.Cu") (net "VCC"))
 (segment (start 120.69 124.46) (end 128.31 124.46) (width 0.2) (layer "F.Cu") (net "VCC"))
 (segment (start 128.31 124.46) (end 135.3625 124.46) (width 0.2) (layer "F.Cu") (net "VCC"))
 (segment (start 185.8973 110.3227) (end 173.4302 110.3227) (width 0.2) (layer "F.Cu") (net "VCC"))
 (segment (start 193.19 109) (end 187.22 109) (width 0.2) (layer "F.Cu") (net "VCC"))
 (segment (start 128.31 110.3317) (end 142.9825 110.3317) (width 0.2) (layer "F.Cu") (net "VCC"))
 (segment (start 142.9825 110.3317) (end 156.5433 110.3317) (width 0.2) (layer "F.Cu") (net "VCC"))
 (segment (start 111.5 111.96) (end 113.1283 110.3317) (width 0.2) (layer "F.Cu") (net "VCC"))
 (segment (start 158.7577 110.3227) (end 157.655 109.22) (width 0.2) (layer "F.Cu") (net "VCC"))
 (segment (start 173.4302 110.3227) (end 172.3275 109.22) (width 0.2) (layer "F.Cu") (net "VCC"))
 (segment (start 179.8904 128.1181) (end 173.4456 128.1181) (width 0.2) (layer "B.Cu") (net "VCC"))
 (segment (start 193.19 120.81) (end 193.19 109) (width 0.2) (layer "B.Cu") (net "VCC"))
 (segment (start 187 127) (end 193.19 120.81) (width 0.2) (layer "B.Cu") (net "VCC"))
 (segment (start 142.9825 127) (end 148.8851 127) (width 0.2) (layer "B.Cu") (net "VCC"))
 (segment (start 129.19 102.5) (end 128.31 103.38) (width 0.2) (layer "B.Cu") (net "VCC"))
 (segment (start 156.5533 128.1017) (end 157.655 127) (width 0.2) (layer "B.Cu") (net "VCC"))
 (segment (start 111.5 111.96) (end 111.5 108.5) (width 0.2) (layer "B.Cu") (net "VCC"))
 (segment (start 135.3625 124.46) (end 137.9025 127) (width 0.2) (layer "B.Cu") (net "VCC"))
 (segment (start 150.035 124.46) (end 148.8851 125.6099) (width 0.2) (layer "B.Cu") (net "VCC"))
 (segment (start 165.2179 128.1181) (end 158.7731 128.1181) (width 0.2) (layer "B.Cu") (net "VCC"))
 (segment (start 166.7918 126.5442) (end 165.2179 128.1181) (width 0.2) (layer "B.Cu") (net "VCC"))
 (segment (start 128.31 127) (end 128.31 124.46) (width 0.2) (layer "B.Cu") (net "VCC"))
 (segment (start 158.7731 128.1181) (end 157.655 127) (width 0.2) (layer "B.Cu") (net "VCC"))
 (segment (start 111.5 108.5) (end 105 102) (width 0.2) (layer "B.Cu") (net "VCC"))
 (segment (start 148.8851 125.6099) (end 148.8851 127) (width 0.2) (layer "B.Cu") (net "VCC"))
 (segment (start 128.31 103.38) (end 128.31 109.22) (width 0.2) (layer "B.Cu") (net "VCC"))
 (segment (start 181.92 127) (end 187 127) (width 0.2) (layer "B.Cu") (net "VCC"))
 (segment (start 148.8851 127) (end 148.8851 127.4208) (width 0.2) (layer "B.Cu") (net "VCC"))
 (segment (start 148.8851 127.4208) (end 149.566 128.1017) (width 0.2) (layer "B.Cu") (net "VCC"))
 (segment (start 166.7918 126.5442) (end 167.2475 127) (width 0.2) (layer "B.Cu") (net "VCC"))
 (segment (start 164.7075 124.46) (end 166.7918 126.5442) (width 0.2) (layer "B.Cu") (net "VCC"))
 (segment (start 167.2475 127) (end 172.3275 127) (width 0.2) (layer "B.Cu") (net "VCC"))
 (segment (start 181.4643 126.5442) (end 181.92 127) (width 0.2) (layer "B.Cu") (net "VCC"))
 (segment (start 179.38 124.46) (end 181.4643 126.5442) (width 0.2) (layer "B.Cu") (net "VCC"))
 (segment (start 181.4643 126.5442) (end 179.8904 128.1181) (width 0.2) (layer "B.Cu") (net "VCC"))
 (segment (start 173.4456 128.1181) (end 172.3275 127) (width 0.2) (layer "B.Cu") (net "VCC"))
 (segment (start 149.566 128.1017) (end 156.5533 128.1017) (width 0.2) (layer "B.Cu") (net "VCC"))
 (segment (start 137.9025 127) (end 142.9825 127) (width 0.2) (layer "B.Cu") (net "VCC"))
 (segment (start 200.5 122) (end 200.5 109.31) (width 0.2) (layer "B.Cu") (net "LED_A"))
 (segment (start 200.5 109.31) (end 200.81 109) (width 0.2) (layer "B.Cu") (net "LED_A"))
 (segment (start 134.66 118.11) (end 136.6325 118.11) (width 0.2) (layer "B.Cu") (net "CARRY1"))
 (segment (start 136.6325 118.11) (end 142.9825 124.46) (width 0.2) (layer "B.Cu") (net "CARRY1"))
 (segment (start 128.31 111.76) (end 134.66 118.11) (width 0.2) (layer "B.Cu") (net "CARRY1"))
 (segment (start 149.3325 118.11) (end 151.305 118.11) (width 0.2) (layer "B.Cu") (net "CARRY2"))
 (segment (start 151.305 118.11) (end 157.655 124.46) (width 0.2) (layer "B.Cu") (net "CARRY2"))
 (segment (start 142.9825 111.76) (end 149.3325 118.11) (width 0.2) (layer "B.Cu") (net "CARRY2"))
 (segment (start 166.7292 118.8617) (end 166.7292 114.7563) (width 0.2) (layer "B.Cu") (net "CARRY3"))
 (segment (start 166.7292 114.7563) (end 165.0029 113.03) (width 0.2) (layer "B.Cu") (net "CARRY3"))
 (segment (start 172.3275 124.46) (end 166.7292 118.8617) (width 0.2) (layer "B.Cu") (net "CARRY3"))
 (segment (start 158.925 113.03) (end 157.655 111.76) (width 0.2) (layer "B.Cu") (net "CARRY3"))
 (segment (start 165.0029 113.03) (end 158.925 113.03) (width 0.2) (layer "B.Cu") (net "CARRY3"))
 (segment (start 187 124.46) (end 181.4017 118.8617) (width 0.2) (layer "B.Cu") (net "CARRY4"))
 (segment (start 181.4017 114.7563) (end 179.6754 113.03) (width 0.2) (layer "B.Cu") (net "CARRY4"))
 (segment (start 173.5975 113.03) (end 172.3275 111.76) (width 0.2) (layer "B.Cu") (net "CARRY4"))
 (segment (start 179.6754 113.03) (end 173.5975 113.03) (width 0.2) (layer "B.Cu") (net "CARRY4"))
 (segment (start 181.4017 118.8617) (end 181.4017 114.7563) (width 0.2) (layer "B.Cu") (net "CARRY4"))
 (segment (start 197.96 122) (end 187.08 122) (width 0.2) (layer "F.Cu") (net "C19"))
 (segment (start 187.08 122) (end 187 121.92) (width 0.2) (layer "F.Cu") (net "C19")))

